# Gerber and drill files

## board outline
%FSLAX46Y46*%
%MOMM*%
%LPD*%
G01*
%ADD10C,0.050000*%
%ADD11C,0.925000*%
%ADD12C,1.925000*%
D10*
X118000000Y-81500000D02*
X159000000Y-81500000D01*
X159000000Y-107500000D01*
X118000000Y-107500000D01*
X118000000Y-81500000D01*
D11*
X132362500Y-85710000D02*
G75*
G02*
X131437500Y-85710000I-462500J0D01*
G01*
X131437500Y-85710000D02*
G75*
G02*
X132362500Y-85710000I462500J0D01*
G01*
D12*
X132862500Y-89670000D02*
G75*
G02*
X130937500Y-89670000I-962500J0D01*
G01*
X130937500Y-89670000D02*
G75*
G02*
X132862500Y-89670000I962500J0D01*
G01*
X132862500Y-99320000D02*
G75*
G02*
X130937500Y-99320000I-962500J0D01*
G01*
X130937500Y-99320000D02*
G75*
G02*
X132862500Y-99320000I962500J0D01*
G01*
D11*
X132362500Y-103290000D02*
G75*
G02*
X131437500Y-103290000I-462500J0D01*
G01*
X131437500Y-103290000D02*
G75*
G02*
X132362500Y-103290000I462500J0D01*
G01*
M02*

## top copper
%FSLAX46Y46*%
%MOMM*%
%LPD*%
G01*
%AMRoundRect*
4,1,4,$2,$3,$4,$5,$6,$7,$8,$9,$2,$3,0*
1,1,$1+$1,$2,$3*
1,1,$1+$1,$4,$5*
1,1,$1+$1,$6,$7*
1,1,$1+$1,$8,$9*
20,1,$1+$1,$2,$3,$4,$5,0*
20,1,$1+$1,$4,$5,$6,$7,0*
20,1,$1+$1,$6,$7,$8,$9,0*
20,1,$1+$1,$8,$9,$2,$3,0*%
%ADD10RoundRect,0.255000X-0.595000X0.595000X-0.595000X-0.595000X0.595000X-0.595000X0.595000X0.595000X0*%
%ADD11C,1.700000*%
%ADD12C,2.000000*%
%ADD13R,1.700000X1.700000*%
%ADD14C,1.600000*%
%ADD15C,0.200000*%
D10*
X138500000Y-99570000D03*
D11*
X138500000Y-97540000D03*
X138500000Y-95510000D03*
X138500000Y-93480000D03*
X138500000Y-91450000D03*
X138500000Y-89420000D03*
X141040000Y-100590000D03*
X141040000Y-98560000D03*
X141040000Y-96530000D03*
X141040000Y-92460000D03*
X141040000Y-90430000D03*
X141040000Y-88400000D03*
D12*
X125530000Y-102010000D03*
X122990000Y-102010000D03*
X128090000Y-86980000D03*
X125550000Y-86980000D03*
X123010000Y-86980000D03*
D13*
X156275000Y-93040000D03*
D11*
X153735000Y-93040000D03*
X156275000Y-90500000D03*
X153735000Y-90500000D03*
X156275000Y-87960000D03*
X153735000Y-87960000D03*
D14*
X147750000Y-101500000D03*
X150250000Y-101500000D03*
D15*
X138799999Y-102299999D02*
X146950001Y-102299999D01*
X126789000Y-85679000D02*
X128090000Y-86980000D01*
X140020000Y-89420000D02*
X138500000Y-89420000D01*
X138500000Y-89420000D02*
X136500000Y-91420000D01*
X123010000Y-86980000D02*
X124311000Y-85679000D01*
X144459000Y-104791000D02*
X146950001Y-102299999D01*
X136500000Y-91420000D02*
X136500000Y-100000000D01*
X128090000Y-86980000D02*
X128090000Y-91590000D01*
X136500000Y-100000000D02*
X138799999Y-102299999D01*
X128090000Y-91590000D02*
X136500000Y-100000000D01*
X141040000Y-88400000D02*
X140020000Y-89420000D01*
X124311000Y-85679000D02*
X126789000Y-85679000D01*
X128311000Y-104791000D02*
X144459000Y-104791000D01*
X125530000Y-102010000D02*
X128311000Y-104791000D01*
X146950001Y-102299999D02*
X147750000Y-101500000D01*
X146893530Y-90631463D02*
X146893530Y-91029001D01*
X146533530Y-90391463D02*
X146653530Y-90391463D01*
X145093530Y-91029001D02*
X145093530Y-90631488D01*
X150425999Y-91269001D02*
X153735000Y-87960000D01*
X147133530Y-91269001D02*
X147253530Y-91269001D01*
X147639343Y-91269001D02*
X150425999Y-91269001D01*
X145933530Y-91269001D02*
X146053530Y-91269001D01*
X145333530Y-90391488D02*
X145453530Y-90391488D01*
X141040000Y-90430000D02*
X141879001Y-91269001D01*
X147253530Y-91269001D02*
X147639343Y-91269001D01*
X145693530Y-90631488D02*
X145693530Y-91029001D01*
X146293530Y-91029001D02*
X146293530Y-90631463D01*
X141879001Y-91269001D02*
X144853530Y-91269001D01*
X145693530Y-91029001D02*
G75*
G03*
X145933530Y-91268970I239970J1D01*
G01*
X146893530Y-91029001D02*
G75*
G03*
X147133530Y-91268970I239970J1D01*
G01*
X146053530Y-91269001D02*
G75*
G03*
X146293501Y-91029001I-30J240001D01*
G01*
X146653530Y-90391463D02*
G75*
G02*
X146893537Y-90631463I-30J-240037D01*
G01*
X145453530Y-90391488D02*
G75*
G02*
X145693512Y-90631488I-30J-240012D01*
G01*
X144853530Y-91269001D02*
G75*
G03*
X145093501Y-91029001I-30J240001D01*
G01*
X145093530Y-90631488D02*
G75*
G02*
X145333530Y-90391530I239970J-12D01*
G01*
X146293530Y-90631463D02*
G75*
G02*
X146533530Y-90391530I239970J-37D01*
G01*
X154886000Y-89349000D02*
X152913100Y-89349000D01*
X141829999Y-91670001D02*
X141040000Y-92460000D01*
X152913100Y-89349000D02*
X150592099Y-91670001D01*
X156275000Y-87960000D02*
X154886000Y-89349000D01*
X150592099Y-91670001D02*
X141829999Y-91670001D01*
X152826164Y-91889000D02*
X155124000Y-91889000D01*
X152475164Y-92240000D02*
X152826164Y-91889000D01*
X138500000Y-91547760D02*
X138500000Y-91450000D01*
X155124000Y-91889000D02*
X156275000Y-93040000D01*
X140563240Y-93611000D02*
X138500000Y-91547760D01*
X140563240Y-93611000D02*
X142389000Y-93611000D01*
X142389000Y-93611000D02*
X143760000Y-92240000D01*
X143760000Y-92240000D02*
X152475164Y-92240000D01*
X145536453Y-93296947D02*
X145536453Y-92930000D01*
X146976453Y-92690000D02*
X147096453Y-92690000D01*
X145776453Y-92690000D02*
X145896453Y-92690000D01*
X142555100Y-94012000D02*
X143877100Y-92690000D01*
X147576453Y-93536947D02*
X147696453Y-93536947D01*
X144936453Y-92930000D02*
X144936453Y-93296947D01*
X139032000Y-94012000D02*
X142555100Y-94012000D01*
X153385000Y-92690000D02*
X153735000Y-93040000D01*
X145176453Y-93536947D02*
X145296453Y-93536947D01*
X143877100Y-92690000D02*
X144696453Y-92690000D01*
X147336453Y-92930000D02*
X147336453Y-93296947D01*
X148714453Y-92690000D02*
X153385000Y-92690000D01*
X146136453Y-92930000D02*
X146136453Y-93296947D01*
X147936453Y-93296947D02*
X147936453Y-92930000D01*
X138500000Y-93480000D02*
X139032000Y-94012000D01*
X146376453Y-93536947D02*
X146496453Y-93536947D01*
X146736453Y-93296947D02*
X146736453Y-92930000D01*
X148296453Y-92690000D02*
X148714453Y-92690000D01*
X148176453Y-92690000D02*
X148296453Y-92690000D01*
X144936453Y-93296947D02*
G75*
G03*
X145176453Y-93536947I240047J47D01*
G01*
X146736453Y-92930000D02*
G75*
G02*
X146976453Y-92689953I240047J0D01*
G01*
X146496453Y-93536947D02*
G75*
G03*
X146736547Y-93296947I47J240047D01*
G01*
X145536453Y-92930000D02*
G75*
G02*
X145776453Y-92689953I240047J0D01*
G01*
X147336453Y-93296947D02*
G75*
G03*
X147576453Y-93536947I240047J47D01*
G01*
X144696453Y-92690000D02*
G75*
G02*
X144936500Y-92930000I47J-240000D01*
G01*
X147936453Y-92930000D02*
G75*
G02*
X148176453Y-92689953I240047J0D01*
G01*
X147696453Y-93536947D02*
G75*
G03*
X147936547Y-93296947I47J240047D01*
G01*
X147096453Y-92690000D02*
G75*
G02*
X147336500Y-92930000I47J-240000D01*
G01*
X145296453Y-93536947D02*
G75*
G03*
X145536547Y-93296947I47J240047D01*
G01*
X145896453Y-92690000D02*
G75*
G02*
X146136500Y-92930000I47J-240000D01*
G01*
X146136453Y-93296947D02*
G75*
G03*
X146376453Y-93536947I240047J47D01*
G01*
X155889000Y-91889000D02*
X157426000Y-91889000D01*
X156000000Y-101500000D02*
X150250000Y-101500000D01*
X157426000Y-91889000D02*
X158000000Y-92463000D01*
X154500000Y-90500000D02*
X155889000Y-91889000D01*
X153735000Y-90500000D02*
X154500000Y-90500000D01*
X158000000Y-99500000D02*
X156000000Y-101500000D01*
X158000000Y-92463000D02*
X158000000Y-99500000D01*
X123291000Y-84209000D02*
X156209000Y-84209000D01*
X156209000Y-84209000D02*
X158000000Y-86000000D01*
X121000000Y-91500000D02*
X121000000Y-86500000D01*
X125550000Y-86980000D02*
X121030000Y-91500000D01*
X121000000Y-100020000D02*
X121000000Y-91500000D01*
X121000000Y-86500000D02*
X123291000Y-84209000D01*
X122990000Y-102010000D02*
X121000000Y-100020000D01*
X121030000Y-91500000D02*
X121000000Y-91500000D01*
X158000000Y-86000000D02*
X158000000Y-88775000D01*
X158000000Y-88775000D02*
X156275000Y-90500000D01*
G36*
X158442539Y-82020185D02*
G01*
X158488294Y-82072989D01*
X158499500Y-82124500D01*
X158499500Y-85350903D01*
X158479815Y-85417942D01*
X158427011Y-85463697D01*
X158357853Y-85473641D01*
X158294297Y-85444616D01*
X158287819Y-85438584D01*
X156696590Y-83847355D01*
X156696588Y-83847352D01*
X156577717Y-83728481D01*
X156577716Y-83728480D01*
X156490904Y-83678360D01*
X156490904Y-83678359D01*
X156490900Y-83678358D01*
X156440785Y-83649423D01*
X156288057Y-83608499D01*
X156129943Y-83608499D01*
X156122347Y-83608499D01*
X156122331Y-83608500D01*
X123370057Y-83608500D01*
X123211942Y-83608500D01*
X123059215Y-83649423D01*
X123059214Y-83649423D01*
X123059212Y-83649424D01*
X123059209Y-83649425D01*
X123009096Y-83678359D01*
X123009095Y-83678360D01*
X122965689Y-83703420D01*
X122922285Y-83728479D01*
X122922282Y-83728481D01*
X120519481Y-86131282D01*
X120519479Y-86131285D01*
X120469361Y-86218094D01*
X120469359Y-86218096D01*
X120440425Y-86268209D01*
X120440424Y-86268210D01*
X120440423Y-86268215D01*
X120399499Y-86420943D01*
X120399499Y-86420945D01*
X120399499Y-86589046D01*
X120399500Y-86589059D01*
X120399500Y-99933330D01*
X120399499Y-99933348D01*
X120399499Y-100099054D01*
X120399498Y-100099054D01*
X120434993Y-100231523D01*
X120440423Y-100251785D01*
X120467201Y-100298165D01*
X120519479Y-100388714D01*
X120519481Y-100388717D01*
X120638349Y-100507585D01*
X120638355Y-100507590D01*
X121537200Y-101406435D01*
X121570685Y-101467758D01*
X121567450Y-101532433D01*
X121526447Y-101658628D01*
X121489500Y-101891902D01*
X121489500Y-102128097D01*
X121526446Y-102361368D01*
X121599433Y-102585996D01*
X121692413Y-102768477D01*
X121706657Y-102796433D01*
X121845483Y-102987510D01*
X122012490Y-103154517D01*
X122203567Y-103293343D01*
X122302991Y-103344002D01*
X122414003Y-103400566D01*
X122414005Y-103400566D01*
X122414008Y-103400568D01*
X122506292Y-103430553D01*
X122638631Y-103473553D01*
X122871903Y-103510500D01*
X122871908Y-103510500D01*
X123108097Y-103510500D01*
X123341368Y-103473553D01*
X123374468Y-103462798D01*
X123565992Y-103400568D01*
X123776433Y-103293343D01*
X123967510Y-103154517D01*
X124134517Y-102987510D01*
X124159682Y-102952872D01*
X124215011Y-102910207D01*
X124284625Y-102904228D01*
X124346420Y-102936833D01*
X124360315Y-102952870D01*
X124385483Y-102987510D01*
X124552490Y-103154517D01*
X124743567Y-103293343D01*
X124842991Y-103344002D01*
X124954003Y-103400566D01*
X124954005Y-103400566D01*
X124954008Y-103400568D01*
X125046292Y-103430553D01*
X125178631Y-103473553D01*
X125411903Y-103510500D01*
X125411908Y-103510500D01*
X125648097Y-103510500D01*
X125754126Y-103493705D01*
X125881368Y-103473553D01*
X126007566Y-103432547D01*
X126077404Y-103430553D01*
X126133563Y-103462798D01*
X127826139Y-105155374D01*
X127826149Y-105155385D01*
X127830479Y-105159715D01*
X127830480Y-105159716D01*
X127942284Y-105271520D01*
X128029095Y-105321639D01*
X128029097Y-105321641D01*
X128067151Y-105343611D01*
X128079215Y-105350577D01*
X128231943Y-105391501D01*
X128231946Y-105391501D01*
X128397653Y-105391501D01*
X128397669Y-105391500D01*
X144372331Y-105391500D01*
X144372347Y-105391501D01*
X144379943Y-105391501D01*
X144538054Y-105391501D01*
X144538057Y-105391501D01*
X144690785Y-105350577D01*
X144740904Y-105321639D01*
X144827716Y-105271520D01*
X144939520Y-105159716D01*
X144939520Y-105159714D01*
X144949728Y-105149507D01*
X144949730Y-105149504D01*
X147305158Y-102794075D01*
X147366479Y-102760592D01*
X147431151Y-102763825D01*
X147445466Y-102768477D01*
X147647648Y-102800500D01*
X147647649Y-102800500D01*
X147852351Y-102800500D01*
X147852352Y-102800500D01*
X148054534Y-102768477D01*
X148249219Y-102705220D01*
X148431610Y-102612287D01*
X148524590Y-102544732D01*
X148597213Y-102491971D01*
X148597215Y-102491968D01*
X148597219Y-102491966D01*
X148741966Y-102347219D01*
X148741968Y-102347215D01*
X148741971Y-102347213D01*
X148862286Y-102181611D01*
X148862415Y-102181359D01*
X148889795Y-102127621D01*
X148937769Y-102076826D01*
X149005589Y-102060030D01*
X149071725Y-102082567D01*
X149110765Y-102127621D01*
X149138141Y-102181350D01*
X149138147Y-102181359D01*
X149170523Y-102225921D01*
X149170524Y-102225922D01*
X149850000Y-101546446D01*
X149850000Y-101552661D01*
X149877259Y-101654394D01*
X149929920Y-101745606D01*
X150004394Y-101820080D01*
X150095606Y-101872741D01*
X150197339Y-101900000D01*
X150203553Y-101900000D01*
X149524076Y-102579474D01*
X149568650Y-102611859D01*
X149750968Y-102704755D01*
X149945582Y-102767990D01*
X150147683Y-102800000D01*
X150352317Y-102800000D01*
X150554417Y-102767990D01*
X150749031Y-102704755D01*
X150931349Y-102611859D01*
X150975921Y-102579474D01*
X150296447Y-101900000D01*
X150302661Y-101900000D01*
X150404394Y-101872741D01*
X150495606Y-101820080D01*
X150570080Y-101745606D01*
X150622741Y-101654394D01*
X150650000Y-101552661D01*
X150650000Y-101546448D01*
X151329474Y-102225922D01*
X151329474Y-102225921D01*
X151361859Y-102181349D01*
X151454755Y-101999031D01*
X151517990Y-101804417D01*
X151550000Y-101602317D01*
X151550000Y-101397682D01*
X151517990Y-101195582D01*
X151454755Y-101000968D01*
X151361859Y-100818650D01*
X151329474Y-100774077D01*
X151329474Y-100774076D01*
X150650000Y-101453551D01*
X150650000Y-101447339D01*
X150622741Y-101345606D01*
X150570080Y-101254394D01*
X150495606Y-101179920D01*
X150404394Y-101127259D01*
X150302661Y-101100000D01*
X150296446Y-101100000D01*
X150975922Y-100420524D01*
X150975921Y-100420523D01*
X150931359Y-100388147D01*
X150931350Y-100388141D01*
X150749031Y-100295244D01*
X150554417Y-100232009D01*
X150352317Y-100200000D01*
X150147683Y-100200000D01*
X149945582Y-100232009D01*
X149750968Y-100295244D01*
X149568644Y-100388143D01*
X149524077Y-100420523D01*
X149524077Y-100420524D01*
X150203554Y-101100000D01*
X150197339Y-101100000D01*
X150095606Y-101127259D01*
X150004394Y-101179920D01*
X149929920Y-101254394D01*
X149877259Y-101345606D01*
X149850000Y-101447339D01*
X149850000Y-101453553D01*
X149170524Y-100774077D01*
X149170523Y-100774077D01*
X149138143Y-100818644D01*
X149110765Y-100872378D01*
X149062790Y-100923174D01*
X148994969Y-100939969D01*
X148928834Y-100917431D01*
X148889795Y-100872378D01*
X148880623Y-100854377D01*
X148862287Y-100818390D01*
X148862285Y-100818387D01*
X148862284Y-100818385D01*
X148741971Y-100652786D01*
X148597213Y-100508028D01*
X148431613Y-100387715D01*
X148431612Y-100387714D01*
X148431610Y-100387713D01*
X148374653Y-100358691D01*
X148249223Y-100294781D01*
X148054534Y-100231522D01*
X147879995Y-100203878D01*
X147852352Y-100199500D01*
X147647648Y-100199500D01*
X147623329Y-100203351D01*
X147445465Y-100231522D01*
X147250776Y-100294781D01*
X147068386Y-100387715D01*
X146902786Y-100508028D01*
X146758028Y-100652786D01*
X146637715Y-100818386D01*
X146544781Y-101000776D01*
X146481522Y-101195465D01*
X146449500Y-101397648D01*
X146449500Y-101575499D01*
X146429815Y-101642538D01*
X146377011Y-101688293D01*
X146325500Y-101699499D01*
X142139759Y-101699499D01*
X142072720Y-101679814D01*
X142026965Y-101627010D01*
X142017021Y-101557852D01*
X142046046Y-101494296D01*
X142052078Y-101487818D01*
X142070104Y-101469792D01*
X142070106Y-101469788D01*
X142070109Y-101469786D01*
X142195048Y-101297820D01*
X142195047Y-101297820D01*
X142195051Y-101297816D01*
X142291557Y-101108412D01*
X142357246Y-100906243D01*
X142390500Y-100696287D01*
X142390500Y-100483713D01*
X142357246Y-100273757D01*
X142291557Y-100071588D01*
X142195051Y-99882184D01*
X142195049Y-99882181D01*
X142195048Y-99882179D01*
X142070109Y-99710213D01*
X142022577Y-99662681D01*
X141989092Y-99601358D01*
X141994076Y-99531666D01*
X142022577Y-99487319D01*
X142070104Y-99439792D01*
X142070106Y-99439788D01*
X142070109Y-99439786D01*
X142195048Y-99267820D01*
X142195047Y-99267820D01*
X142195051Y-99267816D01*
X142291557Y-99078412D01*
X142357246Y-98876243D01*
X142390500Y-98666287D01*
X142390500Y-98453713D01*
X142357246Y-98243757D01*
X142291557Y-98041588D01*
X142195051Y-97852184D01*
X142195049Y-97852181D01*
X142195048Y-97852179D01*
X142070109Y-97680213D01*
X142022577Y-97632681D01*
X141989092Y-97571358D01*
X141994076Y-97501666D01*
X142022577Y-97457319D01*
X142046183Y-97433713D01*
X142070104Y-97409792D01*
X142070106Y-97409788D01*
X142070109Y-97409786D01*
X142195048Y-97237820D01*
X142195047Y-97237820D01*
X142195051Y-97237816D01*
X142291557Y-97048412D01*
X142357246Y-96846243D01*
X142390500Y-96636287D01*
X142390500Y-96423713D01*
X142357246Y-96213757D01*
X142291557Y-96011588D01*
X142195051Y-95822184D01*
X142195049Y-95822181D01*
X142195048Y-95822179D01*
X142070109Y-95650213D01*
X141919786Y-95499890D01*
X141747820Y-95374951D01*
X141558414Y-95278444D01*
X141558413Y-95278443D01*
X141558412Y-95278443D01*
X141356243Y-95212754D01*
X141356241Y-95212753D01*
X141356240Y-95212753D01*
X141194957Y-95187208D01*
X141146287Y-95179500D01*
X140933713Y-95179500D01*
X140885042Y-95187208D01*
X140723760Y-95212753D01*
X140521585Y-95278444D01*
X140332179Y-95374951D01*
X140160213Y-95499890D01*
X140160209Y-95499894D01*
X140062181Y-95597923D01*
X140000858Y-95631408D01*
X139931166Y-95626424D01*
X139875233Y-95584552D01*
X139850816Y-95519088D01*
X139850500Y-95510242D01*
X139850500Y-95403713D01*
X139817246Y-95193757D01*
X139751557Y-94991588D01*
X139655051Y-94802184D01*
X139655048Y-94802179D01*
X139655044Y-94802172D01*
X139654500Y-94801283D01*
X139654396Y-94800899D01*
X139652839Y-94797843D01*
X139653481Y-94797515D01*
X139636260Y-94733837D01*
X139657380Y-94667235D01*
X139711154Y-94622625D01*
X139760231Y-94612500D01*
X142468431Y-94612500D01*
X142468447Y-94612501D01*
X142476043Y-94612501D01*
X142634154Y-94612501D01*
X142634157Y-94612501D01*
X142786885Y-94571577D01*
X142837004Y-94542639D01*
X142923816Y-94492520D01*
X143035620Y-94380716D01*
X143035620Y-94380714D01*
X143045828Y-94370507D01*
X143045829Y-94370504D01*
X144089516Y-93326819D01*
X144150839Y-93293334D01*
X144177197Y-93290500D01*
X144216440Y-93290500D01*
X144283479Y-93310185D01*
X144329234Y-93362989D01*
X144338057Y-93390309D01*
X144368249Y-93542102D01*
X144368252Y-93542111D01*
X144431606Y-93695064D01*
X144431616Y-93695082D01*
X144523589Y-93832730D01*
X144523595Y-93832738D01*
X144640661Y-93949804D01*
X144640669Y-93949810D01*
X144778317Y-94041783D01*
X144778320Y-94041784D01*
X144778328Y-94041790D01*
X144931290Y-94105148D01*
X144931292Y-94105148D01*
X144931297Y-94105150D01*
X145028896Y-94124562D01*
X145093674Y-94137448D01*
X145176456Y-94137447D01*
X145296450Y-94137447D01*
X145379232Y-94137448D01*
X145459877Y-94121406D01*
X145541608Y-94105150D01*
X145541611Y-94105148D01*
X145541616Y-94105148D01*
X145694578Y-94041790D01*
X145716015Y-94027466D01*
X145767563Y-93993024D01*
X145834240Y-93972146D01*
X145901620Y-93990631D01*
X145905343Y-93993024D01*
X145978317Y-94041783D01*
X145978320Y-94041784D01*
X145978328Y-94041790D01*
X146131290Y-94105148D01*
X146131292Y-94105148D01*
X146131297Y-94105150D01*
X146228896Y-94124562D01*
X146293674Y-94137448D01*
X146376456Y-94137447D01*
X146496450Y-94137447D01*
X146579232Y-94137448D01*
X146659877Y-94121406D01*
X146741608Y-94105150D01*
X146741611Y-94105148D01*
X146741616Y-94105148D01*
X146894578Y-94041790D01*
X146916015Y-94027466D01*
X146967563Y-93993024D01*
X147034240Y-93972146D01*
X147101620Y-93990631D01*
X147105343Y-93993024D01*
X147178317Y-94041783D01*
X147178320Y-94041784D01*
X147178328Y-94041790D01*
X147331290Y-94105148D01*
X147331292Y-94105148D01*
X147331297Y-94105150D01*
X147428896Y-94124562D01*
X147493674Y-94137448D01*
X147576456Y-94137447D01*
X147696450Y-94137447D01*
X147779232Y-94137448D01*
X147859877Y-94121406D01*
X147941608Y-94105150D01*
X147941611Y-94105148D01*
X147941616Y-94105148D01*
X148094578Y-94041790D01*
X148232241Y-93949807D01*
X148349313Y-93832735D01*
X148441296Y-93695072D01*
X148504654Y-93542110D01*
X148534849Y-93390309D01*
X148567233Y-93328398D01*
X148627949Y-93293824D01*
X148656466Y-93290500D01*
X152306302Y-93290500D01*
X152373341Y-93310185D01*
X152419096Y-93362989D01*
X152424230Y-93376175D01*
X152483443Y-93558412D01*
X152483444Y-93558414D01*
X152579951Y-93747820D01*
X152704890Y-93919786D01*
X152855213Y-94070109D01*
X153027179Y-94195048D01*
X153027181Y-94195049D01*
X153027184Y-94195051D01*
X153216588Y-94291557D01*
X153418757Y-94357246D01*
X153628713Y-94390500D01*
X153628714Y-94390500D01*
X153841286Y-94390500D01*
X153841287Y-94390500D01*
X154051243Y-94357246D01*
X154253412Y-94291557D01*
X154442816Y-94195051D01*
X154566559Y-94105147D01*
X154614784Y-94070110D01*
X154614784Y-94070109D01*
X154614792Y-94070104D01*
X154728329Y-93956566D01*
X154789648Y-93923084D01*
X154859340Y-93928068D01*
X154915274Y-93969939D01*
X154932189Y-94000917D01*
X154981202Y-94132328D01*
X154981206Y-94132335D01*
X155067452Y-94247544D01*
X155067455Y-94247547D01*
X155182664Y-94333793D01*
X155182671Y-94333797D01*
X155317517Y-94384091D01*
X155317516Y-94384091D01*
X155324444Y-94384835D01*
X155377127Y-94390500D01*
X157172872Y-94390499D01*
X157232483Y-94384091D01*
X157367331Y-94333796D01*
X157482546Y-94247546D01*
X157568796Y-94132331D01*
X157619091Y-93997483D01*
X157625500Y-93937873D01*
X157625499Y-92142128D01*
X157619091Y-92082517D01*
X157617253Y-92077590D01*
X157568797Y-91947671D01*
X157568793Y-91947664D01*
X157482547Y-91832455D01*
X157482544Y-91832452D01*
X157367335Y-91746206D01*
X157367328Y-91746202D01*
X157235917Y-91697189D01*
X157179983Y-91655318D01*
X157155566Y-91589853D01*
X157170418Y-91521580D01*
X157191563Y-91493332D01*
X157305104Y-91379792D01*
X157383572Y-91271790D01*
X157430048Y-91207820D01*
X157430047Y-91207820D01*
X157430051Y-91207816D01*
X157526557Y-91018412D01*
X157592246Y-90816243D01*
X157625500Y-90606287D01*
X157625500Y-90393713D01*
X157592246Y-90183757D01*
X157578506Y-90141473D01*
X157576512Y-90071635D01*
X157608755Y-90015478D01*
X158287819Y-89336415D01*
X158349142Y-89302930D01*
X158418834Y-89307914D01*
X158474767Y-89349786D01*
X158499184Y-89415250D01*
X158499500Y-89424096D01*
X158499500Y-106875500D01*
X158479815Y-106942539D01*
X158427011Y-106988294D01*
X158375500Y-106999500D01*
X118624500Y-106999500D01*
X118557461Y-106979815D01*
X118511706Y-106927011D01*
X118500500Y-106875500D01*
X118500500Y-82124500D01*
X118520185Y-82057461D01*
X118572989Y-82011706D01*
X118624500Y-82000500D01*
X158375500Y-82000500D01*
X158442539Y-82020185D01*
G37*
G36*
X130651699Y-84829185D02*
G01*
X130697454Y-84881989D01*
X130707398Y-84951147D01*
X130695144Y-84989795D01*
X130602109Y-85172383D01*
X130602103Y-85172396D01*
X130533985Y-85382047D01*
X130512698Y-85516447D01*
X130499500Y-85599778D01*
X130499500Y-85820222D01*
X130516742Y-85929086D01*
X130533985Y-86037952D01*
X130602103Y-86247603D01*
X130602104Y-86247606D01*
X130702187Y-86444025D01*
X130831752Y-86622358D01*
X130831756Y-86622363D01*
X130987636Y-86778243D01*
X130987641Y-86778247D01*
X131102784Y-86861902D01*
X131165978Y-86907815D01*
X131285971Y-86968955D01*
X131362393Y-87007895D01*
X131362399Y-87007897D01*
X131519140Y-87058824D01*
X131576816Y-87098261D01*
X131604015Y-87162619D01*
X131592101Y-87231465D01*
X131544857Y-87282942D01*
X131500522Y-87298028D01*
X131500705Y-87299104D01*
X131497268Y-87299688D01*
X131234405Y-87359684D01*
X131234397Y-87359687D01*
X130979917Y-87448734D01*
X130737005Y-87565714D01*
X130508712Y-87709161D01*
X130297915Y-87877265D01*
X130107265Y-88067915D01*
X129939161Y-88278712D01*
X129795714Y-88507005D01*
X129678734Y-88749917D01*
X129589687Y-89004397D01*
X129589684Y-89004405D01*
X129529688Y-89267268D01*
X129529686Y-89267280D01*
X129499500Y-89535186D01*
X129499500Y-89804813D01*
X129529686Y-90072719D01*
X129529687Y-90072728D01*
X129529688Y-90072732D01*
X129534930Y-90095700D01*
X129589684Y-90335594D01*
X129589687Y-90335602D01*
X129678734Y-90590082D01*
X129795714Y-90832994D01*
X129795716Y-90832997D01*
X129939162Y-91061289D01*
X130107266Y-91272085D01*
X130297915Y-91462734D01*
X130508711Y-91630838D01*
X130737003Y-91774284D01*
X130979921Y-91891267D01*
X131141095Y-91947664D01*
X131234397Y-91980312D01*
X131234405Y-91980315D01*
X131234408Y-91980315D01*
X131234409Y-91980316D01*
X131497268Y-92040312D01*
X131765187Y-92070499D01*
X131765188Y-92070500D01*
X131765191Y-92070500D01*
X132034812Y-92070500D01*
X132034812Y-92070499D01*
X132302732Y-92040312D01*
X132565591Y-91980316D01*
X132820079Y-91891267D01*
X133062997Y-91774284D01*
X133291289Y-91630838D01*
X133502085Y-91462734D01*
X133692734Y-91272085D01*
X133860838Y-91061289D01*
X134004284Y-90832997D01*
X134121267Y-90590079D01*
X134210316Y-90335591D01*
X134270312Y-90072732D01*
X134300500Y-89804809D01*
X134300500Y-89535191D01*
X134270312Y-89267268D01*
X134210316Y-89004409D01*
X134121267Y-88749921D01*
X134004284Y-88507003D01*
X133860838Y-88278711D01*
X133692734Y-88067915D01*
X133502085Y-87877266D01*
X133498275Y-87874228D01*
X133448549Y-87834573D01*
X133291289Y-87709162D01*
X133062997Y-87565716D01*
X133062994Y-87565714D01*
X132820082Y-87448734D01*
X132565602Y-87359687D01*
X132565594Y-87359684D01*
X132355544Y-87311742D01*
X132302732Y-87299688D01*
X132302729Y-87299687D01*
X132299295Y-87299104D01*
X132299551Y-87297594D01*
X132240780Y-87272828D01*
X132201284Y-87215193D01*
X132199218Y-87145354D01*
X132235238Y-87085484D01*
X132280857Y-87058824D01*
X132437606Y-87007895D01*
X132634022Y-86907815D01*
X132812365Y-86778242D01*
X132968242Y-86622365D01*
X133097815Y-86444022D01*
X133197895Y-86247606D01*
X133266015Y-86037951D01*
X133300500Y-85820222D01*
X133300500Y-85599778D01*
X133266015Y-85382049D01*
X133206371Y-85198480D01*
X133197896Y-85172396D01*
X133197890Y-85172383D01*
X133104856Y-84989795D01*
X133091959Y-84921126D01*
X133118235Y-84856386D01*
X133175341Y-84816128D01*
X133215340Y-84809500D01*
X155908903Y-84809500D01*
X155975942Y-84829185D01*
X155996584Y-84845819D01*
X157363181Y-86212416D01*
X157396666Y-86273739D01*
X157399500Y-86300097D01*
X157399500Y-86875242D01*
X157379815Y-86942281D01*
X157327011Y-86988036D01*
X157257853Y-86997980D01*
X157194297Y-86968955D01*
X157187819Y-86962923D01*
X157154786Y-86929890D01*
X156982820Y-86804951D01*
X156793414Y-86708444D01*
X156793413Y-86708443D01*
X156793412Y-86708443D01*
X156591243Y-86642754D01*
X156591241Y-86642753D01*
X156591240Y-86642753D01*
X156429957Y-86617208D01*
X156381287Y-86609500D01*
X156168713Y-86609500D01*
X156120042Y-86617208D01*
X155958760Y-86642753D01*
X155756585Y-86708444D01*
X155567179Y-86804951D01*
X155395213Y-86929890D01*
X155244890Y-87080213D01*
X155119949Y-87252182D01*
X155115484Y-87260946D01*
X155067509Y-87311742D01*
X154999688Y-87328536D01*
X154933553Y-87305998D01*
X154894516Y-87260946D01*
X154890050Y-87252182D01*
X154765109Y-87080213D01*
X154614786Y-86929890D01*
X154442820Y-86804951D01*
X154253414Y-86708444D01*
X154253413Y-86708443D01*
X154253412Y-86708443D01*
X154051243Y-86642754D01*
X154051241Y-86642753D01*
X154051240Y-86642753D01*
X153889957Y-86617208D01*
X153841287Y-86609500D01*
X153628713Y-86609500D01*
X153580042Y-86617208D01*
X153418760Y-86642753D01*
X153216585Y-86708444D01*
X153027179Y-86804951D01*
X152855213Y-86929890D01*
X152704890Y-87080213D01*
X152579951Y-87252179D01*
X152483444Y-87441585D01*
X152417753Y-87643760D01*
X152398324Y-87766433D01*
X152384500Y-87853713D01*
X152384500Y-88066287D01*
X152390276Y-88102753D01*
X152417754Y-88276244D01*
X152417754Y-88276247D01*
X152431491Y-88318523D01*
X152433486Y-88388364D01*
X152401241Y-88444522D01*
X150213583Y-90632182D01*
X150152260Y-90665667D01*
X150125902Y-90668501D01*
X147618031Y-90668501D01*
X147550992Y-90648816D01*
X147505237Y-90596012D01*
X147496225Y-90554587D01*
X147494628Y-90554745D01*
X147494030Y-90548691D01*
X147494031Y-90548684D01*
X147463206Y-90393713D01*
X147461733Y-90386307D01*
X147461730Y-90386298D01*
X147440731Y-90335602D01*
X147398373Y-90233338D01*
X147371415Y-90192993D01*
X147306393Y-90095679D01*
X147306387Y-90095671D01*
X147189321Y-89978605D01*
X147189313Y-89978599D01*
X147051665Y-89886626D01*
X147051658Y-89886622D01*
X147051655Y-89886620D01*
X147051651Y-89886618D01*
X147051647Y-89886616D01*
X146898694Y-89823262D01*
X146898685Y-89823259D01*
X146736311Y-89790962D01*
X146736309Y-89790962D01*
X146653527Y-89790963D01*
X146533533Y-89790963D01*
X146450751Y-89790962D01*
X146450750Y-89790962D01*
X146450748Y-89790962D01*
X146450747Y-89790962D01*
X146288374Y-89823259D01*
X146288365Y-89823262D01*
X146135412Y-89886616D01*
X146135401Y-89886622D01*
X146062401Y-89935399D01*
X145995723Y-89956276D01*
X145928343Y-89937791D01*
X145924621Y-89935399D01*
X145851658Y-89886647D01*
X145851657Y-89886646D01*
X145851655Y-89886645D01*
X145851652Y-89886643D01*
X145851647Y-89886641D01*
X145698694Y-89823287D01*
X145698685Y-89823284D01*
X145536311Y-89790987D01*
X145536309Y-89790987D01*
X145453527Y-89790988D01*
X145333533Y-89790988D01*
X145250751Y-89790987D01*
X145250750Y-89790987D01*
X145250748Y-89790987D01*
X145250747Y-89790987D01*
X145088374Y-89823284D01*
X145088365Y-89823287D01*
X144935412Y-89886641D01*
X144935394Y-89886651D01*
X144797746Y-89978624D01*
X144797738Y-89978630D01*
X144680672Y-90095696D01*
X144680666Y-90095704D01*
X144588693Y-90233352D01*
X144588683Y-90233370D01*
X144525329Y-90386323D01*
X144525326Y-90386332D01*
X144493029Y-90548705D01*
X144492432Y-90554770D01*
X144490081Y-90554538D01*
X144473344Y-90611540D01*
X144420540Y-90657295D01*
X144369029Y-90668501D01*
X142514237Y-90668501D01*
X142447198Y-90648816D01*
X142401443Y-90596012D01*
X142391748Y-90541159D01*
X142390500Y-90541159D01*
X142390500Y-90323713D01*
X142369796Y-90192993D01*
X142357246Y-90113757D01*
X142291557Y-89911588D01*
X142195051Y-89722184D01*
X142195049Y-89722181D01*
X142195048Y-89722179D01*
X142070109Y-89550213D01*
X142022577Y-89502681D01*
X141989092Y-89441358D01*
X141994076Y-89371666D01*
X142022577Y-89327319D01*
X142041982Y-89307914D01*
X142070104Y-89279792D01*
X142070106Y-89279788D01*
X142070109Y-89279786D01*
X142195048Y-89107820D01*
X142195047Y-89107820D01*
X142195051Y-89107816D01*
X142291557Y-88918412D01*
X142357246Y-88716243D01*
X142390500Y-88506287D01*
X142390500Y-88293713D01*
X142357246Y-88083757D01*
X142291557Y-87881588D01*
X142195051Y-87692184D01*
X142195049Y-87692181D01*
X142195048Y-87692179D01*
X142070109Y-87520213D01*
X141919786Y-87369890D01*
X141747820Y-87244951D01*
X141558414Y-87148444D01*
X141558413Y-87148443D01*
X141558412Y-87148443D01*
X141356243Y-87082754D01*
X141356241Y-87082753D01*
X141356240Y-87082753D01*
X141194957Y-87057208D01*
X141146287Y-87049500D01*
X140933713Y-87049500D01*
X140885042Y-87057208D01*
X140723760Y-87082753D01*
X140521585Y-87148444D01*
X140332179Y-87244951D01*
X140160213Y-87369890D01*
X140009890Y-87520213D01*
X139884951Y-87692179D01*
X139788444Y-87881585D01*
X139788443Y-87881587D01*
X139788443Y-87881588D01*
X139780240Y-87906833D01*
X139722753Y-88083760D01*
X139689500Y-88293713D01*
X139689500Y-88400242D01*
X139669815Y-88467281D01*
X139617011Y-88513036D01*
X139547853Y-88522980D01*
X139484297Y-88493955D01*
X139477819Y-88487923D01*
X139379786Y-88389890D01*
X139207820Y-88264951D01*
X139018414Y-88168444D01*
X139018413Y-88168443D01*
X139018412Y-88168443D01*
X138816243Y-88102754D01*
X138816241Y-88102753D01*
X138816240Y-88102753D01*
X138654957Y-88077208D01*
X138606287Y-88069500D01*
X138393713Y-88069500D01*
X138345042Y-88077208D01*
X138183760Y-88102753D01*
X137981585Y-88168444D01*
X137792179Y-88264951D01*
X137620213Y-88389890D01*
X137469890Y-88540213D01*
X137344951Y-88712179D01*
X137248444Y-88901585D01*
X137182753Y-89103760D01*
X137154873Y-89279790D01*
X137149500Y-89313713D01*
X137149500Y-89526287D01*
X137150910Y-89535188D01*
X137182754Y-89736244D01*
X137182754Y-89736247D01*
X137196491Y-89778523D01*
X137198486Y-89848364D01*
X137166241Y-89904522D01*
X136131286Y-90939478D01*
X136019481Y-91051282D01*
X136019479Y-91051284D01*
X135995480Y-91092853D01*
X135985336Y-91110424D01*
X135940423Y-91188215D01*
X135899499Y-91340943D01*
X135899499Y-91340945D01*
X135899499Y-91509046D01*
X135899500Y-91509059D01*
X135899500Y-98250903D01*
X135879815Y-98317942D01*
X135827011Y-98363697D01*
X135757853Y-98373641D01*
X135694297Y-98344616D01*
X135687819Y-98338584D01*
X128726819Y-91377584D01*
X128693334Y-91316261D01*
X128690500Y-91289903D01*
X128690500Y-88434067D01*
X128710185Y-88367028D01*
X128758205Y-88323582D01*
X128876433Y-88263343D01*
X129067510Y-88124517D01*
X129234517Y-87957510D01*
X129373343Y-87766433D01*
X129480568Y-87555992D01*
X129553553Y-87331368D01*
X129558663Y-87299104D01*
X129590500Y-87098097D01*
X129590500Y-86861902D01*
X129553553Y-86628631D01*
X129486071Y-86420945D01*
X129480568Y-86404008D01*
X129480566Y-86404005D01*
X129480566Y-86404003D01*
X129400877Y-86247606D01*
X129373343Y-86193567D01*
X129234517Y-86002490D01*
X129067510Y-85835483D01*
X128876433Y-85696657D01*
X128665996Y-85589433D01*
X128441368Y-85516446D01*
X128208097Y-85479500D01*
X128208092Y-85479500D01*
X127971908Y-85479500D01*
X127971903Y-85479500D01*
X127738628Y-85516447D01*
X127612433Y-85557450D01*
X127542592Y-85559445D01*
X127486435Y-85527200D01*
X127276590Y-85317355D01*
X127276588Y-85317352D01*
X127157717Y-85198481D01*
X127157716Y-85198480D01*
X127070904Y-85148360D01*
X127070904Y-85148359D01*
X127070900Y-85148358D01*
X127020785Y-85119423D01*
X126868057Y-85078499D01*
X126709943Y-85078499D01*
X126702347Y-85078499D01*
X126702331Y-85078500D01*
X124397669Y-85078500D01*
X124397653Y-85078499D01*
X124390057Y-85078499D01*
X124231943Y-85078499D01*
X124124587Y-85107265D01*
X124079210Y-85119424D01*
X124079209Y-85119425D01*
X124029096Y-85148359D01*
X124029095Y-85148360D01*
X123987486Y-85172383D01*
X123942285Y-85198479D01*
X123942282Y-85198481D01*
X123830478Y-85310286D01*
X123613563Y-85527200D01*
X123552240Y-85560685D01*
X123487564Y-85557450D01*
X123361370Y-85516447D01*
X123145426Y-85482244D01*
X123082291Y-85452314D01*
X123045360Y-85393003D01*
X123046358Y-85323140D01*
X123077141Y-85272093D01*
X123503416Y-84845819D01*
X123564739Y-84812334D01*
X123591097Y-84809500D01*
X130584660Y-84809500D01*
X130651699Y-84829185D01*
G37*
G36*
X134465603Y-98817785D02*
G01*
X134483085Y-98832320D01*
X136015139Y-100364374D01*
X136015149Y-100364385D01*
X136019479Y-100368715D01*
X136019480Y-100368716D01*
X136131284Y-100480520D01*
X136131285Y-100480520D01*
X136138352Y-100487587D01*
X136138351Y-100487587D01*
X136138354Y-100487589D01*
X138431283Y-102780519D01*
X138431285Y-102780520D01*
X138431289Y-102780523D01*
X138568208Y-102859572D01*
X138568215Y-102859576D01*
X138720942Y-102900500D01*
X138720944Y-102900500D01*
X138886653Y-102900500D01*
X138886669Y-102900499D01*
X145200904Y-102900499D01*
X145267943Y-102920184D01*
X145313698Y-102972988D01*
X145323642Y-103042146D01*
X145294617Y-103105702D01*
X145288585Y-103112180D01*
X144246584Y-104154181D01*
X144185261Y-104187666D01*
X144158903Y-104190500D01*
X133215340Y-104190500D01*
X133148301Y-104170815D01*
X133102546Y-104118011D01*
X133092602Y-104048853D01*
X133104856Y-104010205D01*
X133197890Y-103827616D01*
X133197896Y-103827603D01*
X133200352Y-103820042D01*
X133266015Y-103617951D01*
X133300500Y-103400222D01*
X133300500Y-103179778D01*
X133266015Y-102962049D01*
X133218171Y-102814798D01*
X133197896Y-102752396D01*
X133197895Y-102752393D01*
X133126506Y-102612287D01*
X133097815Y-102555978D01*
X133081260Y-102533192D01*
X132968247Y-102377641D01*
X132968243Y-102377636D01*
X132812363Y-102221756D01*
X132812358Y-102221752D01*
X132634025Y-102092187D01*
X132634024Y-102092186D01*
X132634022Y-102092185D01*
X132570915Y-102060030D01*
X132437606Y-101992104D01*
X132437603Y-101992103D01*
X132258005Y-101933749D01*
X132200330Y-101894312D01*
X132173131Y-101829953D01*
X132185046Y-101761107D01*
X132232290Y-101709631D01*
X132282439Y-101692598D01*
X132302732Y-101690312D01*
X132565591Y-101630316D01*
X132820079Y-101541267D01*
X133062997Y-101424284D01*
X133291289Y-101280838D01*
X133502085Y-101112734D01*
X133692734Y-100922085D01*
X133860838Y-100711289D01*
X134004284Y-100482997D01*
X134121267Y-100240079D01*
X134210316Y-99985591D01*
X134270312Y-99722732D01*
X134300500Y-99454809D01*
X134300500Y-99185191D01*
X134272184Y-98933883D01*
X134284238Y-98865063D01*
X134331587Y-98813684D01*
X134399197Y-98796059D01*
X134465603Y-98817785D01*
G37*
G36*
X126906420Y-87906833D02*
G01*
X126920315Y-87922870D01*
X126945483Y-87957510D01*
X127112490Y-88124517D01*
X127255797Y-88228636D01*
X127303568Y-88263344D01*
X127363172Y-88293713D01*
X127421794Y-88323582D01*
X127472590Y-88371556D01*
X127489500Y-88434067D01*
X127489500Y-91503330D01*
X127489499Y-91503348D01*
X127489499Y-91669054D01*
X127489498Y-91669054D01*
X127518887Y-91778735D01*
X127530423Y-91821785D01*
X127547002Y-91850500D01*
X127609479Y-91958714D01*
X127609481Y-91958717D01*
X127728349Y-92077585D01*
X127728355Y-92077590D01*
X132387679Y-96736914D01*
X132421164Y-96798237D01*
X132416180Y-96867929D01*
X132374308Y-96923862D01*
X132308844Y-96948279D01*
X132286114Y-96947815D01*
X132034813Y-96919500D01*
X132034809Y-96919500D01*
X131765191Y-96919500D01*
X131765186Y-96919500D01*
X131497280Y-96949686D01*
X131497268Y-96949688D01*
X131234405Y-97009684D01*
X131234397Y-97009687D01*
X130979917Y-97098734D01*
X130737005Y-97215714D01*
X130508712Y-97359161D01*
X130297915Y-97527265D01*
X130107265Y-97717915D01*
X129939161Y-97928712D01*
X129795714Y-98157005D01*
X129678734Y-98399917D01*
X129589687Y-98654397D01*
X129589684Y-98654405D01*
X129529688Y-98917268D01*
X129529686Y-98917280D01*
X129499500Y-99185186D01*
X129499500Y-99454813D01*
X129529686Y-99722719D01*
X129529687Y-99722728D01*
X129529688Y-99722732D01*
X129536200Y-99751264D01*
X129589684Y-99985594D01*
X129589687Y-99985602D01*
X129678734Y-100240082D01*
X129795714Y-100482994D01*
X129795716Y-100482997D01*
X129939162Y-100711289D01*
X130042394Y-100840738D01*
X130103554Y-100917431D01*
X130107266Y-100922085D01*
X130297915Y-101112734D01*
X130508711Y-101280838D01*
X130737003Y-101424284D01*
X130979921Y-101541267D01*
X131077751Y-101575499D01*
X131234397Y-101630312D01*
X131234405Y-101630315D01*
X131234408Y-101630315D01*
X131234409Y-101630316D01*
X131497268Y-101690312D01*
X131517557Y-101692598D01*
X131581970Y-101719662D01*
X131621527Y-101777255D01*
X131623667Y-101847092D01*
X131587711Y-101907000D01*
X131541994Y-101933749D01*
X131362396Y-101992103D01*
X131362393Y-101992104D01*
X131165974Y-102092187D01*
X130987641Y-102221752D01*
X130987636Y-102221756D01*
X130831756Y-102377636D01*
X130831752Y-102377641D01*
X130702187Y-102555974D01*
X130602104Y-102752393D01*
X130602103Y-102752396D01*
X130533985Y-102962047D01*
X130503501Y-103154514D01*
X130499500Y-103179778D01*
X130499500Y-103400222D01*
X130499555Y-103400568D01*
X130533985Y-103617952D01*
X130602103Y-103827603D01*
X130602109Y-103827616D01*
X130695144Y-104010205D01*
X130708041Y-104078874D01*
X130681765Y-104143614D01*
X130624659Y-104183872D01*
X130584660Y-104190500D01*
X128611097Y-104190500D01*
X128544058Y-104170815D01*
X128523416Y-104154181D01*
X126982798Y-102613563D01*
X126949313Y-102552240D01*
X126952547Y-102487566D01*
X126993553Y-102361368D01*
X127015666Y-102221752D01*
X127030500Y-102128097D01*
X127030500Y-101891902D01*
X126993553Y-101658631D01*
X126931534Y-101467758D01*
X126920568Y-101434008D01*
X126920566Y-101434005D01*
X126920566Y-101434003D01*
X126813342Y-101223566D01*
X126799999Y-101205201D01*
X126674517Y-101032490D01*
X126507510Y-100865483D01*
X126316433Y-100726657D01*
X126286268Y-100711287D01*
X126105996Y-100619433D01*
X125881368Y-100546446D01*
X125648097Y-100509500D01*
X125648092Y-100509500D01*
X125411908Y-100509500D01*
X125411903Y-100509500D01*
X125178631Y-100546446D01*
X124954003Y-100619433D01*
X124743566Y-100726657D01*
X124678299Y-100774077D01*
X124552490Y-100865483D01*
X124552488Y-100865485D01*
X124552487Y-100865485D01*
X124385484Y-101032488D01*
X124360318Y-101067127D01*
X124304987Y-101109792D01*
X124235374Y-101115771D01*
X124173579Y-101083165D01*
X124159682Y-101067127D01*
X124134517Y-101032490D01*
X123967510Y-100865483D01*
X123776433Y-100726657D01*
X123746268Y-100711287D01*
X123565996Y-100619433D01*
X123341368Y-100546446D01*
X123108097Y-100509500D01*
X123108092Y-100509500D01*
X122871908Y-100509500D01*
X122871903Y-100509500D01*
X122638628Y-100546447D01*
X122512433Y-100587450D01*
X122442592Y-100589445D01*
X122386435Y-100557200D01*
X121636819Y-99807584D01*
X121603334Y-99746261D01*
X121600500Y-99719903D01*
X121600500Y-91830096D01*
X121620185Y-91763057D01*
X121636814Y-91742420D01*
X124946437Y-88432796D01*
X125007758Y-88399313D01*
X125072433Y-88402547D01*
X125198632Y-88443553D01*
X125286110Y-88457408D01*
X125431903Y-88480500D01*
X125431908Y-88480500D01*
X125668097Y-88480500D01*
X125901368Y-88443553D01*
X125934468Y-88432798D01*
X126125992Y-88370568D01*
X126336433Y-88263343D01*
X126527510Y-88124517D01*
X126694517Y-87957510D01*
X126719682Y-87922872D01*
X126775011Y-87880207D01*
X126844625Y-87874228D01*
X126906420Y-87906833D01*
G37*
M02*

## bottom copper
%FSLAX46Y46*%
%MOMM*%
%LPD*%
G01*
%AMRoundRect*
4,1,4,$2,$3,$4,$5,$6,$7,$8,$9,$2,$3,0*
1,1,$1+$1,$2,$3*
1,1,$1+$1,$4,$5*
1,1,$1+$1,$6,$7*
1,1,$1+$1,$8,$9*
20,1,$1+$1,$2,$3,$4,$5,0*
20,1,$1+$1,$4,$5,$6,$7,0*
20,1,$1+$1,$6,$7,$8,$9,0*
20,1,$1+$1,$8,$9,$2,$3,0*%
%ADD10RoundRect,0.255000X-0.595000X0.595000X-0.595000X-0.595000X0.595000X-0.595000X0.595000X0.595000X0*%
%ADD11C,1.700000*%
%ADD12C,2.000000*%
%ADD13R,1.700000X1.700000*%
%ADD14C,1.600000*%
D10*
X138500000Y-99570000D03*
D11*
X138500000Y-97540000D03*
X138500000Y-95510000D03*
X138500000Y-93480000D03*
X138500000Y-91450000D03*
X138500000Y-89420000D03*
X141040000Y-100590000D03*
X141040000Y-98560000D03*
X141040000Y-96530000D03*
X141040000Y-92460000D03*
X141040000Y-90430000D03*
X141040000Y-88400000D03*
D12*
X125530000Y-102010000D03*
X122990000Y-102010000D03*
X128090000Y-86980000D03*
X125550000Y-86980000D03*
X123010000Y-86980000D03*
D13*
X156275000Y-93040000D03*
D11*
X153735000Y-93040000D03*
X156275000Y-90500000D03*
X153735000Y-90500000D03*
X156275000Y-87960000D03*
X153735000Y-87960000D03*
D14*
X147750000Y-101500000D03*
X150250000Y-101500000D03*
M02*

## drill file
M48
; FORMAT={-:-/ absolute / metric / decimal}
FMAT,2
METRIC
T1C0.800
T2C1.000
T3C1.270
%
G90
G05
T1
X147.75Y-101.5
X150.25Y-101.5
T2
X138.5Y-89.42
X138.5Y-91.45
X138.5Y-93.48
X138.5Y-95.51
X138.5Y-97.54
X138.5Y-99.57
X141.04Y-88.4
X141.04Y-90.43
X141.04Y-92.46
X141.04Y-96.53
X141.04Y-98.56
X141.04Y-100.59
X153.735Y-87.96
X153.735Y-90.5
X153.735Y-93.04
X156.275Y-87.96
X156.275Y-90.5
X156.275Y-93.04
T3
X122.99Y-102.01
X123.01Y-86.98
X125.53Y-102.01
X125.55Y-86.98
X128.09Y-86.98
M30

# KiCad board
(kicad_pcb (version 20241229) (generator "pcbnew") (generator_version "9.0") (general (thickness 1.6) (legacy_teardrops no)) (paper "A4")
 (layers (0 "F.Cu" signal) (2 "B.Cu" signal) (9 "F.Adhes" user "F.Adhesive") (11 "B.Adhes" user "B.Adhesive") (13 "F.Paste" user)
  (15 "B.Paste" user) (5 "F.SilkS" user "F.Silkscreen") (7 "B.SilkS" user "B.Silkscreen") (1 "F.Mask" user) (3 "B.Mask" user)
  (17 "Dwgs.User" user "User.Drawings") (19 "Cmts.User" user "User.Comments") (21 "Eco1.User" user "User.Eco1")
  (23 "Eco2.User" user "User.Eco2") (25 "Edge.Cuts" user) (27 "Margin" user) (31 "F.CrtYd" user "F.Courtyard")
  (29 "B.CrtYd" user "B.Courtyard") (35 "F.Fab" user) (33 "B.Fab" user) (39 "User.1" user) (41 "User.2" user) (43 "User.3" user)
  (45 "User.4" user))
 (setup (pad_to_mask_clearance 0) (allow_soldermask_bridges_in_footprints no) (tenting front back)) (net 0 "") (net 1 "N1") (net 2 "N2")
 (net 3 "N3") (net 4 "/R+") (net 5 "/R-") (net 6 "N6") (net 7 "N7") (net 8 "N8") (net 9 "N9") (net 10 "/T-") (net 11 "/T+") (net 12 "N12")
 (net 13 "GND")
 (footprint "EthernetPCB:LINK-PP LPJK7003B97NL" (layer "F.Cu") (at 138.5 99.57 -90)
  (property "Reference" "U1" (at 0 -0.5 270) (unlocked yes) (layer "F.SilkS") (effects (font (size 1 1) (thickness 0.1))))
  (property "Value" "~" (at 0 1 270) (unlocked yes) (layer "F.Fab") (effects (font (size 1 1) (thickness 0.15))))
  (fp_circle (center -13.86 6.6) (end -12.96 6.6) (stroke (width 0.05) (type solid)) (fill yes) (layer "Edge.Cuts"))
  (fp_circle (center -9.9 6.6) (end -8 6.6) (stroke (width 0.05) (type solid)) (fill yes) (layer "Edge.Cuts"))
  (fp_circle (center -0.25 6.6) (end 1.65 6.6) (stroke (width 0.05) (type solid)) (fill yes) (layer "Edge.Cuts"))
  (fp_circle (center 3.72 6.6) (end 4.62 6.6) (stroke (width 0.05) (type solid)) (fill yes) (layer "Edge.Cuts"))
  (pad "1" thru_hole roundrect (at 0 0 270) (size 1.7 1.7) (drill 1) (layers "*.Cu" "*.Mask") (remove_unused_layers no)
   (roundrect_rratio 0.15) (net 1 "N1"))
  (pad "2" thru_hole circle (at -2.03 0 270) (size 1.7 1.7) (drill 1) (layers "*.Cu" "*.Mask") (remove_unused_layers no) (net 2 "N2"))
  (pad "3" thru_hole circle (at -4.06 0 270) (size 1.7 1.7) (drill 1) (layers "*.Cu" "*.Mask") (remove_unused_layers no) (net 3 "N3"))
  (pad "4" thru_hole circle (at -6.09 0 270) (size 1.7 1.7) (drill 1) (layers "*.Cu" "*.Mask") (remove_unused_layers no) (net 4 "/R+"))
  (pad "5" thru_hole circle (at -8.12 0 270) (size 1.7 1.7) (drill 1) (layers "*.Cu" "*.Mask") (remove_unused_layers no) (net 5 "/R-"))
  (pad "6" thru_hole circle (at -10.15 0 270) (size 1.7 1.7) (drill 1) (layers "*.Cu" "*.Mask") (remove_unused_layers no) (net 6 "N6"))
  (pad "7" thru_hole circle (at 1.02 -2.54 270) (size 1.7 1.7) (drill 1) (layers "*.Cu" "*.Mask") (remove_unused_layers no) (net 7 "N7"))
  (pad "8" thru_hole circle (at -1.01 -2.54 270) (size 1.7 1.7) (drill 1) (layers "*.Cu" "*.Mask") (remove_unused_layers no) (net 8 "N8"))
  (pad "9" thru_hole circle (at -3.04 -2.54 270) (size 1.7 1.7) (drill 1) (layers "*.Cu" "*.Mask") (remove_unused_layers no) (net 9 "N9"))
  (pad "10" thru_hole circle (at -7.11 -2.54 270) (size 1.7 1.7) (drill 1) (layers "*.Cu" "*.Mask") (remove_unused_layers no) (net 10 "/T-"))
  (pad "11" thru_hole circle (at -9.14 -2.54 270) (size 1.7 1.7) (drill 1) (layers "*.Cu" "*.Mask") (remove_unused_layers no) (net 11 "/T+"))
  (pad "12" thru_hole circle (at -11.17 -2.54 270) (size 1.7 1.7) (drill 1) (layers "*.Cu" "*.Mask") (remove_unused_layers no) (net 6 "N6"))
  (pad "13" thru_hole circle (at 2.44 12.97 270) (size 2 2) (drill 1.27) (layers "*.Cu" "*.Mask") (remove_unused_layers no) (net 6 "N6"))
  (pad "14" thru_hole circle (at 2.44 15.51 270) (size 2 2) (drill 1.27) (layers "*.Cu" "*.Mask") (remove_unused_layers no) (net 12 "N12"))
  (pad "15" thru_hole circle (at -12.59 10.41 270) (size 2 2) (drill 1.27) (layers "*.Cu" "*.Mask") (remove_unused_layers no) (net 6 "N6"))
  (pad "16" thru_hole circle (at -12.59 12.95 270) (size 2 2) (drill 1.27) (layers "*.Cu" "*.Mask") (remove_unused_layers no) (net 12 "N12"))
  (pad "17" thru_hole circle (at -12.59 15.49 270) (size 2 2) (drill 1.27) (layers "*.Cu" "*.Mask") (remove_unused_layers no) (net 6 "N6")))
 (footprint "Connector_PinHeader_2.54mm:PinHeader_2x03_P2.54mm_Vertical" (layer "F.Cu") (at 156.275 93.04 180)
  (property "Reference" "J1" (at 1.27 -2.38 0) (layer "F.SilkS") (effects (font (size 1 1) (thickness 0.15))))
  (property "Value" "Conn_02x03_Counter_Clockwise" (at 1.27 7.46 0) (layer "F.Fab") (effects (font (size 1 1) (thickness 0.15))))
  (pad "1" thru_hole rect (at 0 0 180) (size 1.7 1.7) (drill 1) (layers "*.Cu" "*.Mask") (remove_unused_layers no) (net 5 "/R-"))
  (pad "2" thru_hole circle (at 2.54 0 180) (size 1.7 1.7) (drill 1) (layers "*.Cu" "*.Mask") (remove_unused_layers no) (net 4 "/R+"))
  (pad "3" thru_hole circle (at 0 2.54 180) (size 1.7 1.7) (drill 1) (layers "*.Cu" "*.Mask") (remove_unused_layers no) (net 12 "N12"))
  (pad "4" thru_hole circle (at 2.54 2.54 180) (size 1.7 1.7) (drill 1) (layers "*.Cu" "*.Mask") (remove_unused_layers no) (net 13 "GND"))
  (pad "5" thru_hole circle (at 0 5.08 180) (size 1.7 1.7) (drill 1) (layers "*.Cu" "*.Mask") (remove_unused_layers no) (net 10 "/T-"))
  (pad "6" thru_hole circle (at 2.54 5.08 180) (size 1.7 1.7) (drill 1) (layers "*.Cu" "*.Mask") (remove_unused_layers no) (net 11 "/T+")))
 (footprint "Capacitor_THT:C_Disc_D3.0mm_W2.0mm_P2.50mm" (layer "F.Cu") (at 147.75 101.5)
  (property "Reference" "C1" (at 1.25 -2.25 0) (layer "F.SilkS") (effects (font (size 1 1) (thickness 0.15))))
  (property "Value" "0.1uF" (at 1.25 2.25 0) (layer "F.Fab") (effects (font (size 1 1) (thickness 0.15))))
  (pad "1" thru_hole circle (at 0 0) (size 1.6 1.6) (drill 0.8) (layers "*.Cu" "*.Mask") (remove_unused_layers no) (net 6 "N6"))
  (pad "2" thru_hole circle (at 2.5 0) (size 1.6 1.6) (drill 0.8) (layers "*.Cu" "*.Mask") (remove_unused_layers no) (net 13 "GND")))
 (gr_rect (start 118 81.5) (end 159 107.5) (stroke (width 0.05) (type solid)) (fill no) (layer "Edge.Cuts"))
 (segment (start 138.799999 102.299999) (end 146.950001 102.299999) (width 0.2) (layer "F.Cu") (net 6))
 (segment (start 126.789 85.679) (end 128.09 86.98) (width 0.2) (layer "F.Cu") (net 6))
 (segment (start 140.02 89.42) (end 138.5 89.42) (width 0.2) (layer "F.Cu") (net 6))
 (segment (start 138.5 89.42) (end 136.5 91.42) (width 0.2) (layer "F.Cu") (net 6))
 (segment (start 123.01 86.98) (end 124.311 85.679) (width 0.2) (layer "F.Cu") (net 6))
 (segment (start 144.459 104.791) (end 146.950001 102.299999) (width 0.2) (layer "F.Cu") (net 6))
 (segment (start 136.5 91.42) (end 136.5 100) (width 0.2) (layer "F.Cu") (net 6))
 (segment (start 128.09 86.98) (end 128.09 91.59) (width 0.2) (layer "F.Cu") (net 6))
 (segment (start 136.5 100) (end 138.799999 102.299999) (width 0.2) (layer "F.Cu") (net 6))
 (segment (start 128.09 91.59) (end 136.5 100) (width 0.2) (layer "F.Cu") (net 6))
 (segment (start 141.04 88.4) (end 140.02 89.42) (width 0.2) (layer "F.Cu") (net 6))
 (segment (start 124.311 85.679) (end 126.789 85.679) (width 0.2) (layer "F.Cu") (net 6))
 (segment (start 128.311 104.791) (end 144.459 104.791) (width 0.2) (layer "F.Cu") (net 6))
 (segment (start 125.53 102.01) (end 128.311 104.791) (width 0.2) (layer "F.Cu") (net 6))
 (segment (start 146.950001 102.299999) (end 147.75 101.5) (width 0.2) (layer "F.Cu") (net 6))
 (segment (start 146.89353 90.631463) (end 146.89353 91.029001) (width 0.2) (layer "F.Cu") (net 11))
 (segment (start 146.53353 90.391463) (end 146.65353 90.391463) (width 0.2) (layer "F.Cu") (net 11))
 (segment (start 145.09353 91.029001) (end 145.09353 90.631488) (width 0.2) (layer "F.Cu") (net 11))
 (segment (start 150.425999 91.269001) (end 153.735 87.96) (width 0.2) (layer "F.Cu") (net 11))
 (segment (start 147.13353 91.269001) (end 147.25353 91.269001) (width 0.2) (layer "F.Cu") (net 11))
 (segment (start 147.639343 91.269001) (end 150.425999 91.269001) (width 0.2) (layer "F.Cu") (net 11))
 (segment (start 145.93353 91.269001) (end 146.05353 91.269001) (width 0.2) (layer "F.Cu") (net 11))
 (segment (start 145.33353 90.391488) (end 145.45353 90.391488) (width 0.2) (layer "F.Cu") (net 11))
 (segment (start 141.04 90.43) (end 141.879001 91.269001) (width 0.2) (layer "F.Cu") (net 11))
 (segment (start 147.25353 91.269001) (end 147.639343 91.269001) (width 0.2) (layer "F.Cu") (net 11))
 (segment (start 145.69353 90.631488) (end 145.69353 91.029001) (width 0.2) (layer "F.Cu") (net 11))
 (segment (start 146.29353 91.029001) (end 146.29353 90.631463) (width 0.2) (layer "F.Cu") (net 11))
 (segment (start 141.879001 91.269001) (end 144.85353 91.269001) (width 0.2) (layer "F.Cu") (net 11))
 (arc (start 145.69353 91.029001) (mid 145.763824 91.198707) (end 145.93353 91.269001) (width 0.2) (layer "F.Cu") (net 11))
 (arc (start 146.89353 91.029001) (mid 146.963824 91.198707) (end 147.13353 91.269001) (width 0.2) (layer "F.Cu") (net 11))
 (arc (start 146.05353 91.269001) (mid 146.223236 91.198707) (end 146.29353 91.029001) (width 0.2) (layer "F.Cu") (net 11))
 (arc (start 146.65353 90.391463) (mid 146.823236 90.461757) (end 146.89353 90.631463) (width 0.2) (layer "F.Cu") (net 11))
 (arc (start 145.45353 90.391488) (mid 145.623236 90.461782) (end 145.69353 90.631488) (width 0.2) (layer "F.Cu") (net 11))
 (arc (start 144.85353 91.269001) (mid 145.023236 91.198707) (end 145.09353 91.029001) (width 0.2) (layer "F.Cu") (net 11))
 (arc (start 145.09353 90.631488) (mid 145.163824 90.461782) (end 145.33353 90.391488) (width 0.2) (layer "F.Cu") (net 11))
 (arc (start 146.29353 90.631463) (mid 146.363824 90.461757) (end 146.53353 90.391463) (width 0.2) (layer "F.Cu") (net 11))
 (segment (start 154.886 89.349) (end 152.9131 89.349) (width 0.2) (layer "F.Cu") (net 10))
 (segment (start 141.829999 91.670001) (end 141.04 92.46) (width 0.2) (layer "F.Cu") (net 10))
 (segment (start 152.9131 89.349) (end 150.592099 91.670001) (width 0.2) (layer "F.Cu") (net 10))
 (segment (start 156.275 87.96) (end 154.886 89.349) (width 0.2) (layer "F.Cu") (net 10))
 (segment (start 150.592099 91.670001) (end 141.829999 91.670001) (width 0.2) (layer "F.Cu") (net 10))
 (segment (start 152.826164 91.889) (end 155.124 91.889) (width 0.2) (layer "F.Cu") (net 5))
 (segment (start 152.475164 92.24) (end 152.826164 91.889) (width 0.2) (layer "F.Cu") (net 5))
 (segment (start 138.5 91.54776) (end 138.5 91.45) (width 0.2) (layer "F.Cu") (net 5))
 (segment (start 155.124 91.889) (end 156.275 93.04) (width 0.2) (layer "F.Cu") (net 5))
 (segment (start 140.56324 93.611) (end 138.5 91.54776) (width 0.2) (layer "F.Cu") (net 5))
 (segment (start 140.56324 93.611) (end 142.389 93.611) (width 0.2) (layer "F.Cu") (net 5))
 (segment (start 142.389 93.611) (end 143.76 92.24) (width 0.2) (layer "F.Cu") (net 5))
 (segment (start 143.76 92.24) (end 152.475164 92.24) (width 0.2) (layer "F.Cu") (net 5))
 (segment (start 145.536453 93.296947) (end 145.536453 92.93) (width 0.2) (layer "F.Cu") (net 4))
 (segment (start 146.976453 92.69) (end 147.096453 92.69) (width 0.2) (layer "F.Cu") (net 4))
 (segment (start 145.776453 92.69) (end 145.896453 92.69) (width 0.2) (layer "F.Cu") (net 4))
 (segment (start 142.5551 94.012) (end 143.8771 92.69) (width 0.2) (layer "F.Cu") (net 4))
 (segment (start 147.576453 93.536947) (end 147.696453 93.536947) (width 0.2) (layer "F.Cu") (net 4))
 (segment (start 144.936453 92.93) (end 144.936453 93.296947) (width 0.2) (layer "F.Cu") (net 4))
 (segment (start 139.032 94.012) (end 142.5551 94.012) (width 0.2) (layer "F.Cu") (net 4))
 (segment (start 153.385 92.69) (end 153.735 93.04) (width 0.2) (layer "F.Cu") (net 4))
 (segment (start 145.176453 93.536947) (end 145.296453 93.536947) (width 0.2) (layer "F.Cu") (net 4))
 (segment (start 143.8771 92.69) (end 144.696453 92.69) (width 0.2) (layer "F.Cu") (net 4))
 (segment (start 147.336453 92.93) (end 147.336453 93.296947) (width 0.2) (layer "F.Cu") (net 4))
 (segment (start 148.714453 92.69) (end 153.385 92.69) (width 0.2) (layer "F.Cu") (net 4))
 (segment (start 146.136453 92.93) (end 146.136453 93.296947) (width 0.2) (layer "F.Cu") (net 4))
 (segment (start 147.936453 93.296947) (end 147.936453 92.93) (width 0.2) (layer "F.Cu") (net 4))
 (segment (start 138.5 93.48) (end 139.032 94.012) (width 0.2) (layer "F.Cu") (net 4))
 (segment (start 146.376453 93.536947) (end 146.496453 93.536947) (width 0.2) (layer "F.Cu") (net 4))
 (segment (start 146.736453 93.296947) (end 146.736453 92.93) (width 0.2) (layer "F.Cu") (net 4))
 (segment (start 148.296453 92.69) (end 148.714453 92.69) (width 0.2) (layer "F.Cu") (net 4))
 (segment (start 148.176453 92.69) (end 148.296453 92.69) (width 0.2) (layer "F.Cu") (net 4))
 (arc (start 144.936453 93.296947) (mid 145.006747 93.466653) (end 145.176453 93.536947) (width 0.2) (layer "F.Cu") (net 4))
 (arc (start 146.736453 92.93) (mid 146.806747 92.760294) (end 146.976453 92.69) (width 0.2) (layer "F.Cu") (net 4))
 (arc (start 146.496453 93.536947) (mid 146.666159 93.466653) (end 146.736453 93.296947) (width 0.2) (layer "F.Cu") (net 4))
 (arc (start 145.536453 92.93) (mid 145.606747 92.760294) (end 145.776453 92.69) (width 0.2) (layer "F.Cu") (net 4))
 (arc (start 147.336453 93.296947) (mid 147.406747 93.466653) (end 147.576453 93.536947) (width 0.2) (layer "F.Cu") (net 4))
 (arc (start 144.696453 92.69) (mid 144.866159 92.760294) (end 144.936453 92.93) (width 0.2) (layer "F.Cu") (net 4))
 (arc (start 147.936453 92.93) (mid 148.006747 92.760294) (end 148.176453 92.69) (width 0.2) (layer "F.Cu") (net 4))
 (arc (start 147.696453 93.536947) (mid 147.866159 93.466653) (end 147.936453 93.296947) (width 0.2) (layer "F.Cu") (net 4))
 (arc (start 147.096453 92.69) (mid 147.266159 92.760294) (end 147.336453 92.93) (width 0.2) (layer "F.Cu") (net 4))
 (arc (start 145.296453 93.536947) (mid 145.466159 93.466653) (end 145.536453 93.296947) (width 0.2) (layer "F.Cu") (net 4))
 (arc (start 145.896453 92.69) (mid 146.066159 92.760294) (end 146.136453 92.93) (width 0.2) (layer "F.Cu") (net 4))
 (arc (start 146.136453 93.296947) (mid 146.206747 93.466653) (end 146.376453 93.536947) (width 0.2) (layer "F.Cu") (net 4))
 (segment (start 155.889 91.889) (end 157.426 91.889) (width 0.2) (layer "F.Cu") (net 13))
 (segment (start 156 101.5) (end 150.25 101.5) (width 0.2) (layer "F.Cu") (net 13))
 (segment (start 157.426 91.889) (end 158 92.463) (width 0.2) (layer "F.Cu") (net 13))
 (segment (start 154.5 90.5) (end 155.889 91.889) (width 0.2) (layer "F.Cu") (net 13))
 (segment (start 153.735 90.5) (end 154.5 90.5) (width 0.2) (layer "F.Cu") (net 13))
 (segment (start 158 99.5) (end 156 101.5) (width 0.2) (layer "F.Cu") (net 13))
 (segment (start 158 92.463) (end 158 99.5) (width 0.2) (layer "F.Cu") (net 13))
 (segment (start 123.291 84.209) (end 156.209 84.209) (width 0.2) (layer "F.Cu") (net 12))
 (segment (start 156.209 84.209) (end 158 86) (width 0.2) (layer "F.Cu") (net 12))
 (segment (start 121 91.5) (end 121 86.5) (width 0.2) (layer "F.Cu") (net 12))
 (segment (start 125.55 86.98) (end 121.03 91.5) (width 0.2) (layer "F.Cu") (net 12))
 (segment (start 121 100.02) (end 121 91.5) (width 0.2) (layer "F.Cu") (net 12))
 (segment (start 121 86.5) (end 123.291 84.209) (width 0.2) (layer "F.Cu") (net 12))
 (segment (start 122.99 102.01) (end 121 100.02) (width 0.2) (layer "F.Cu") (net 12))
 (segment (start 121.03 91.5) (end 121 91.5) (width 0.2) (layer "F.Cu") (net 12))
 (segment (start 158 86) (end 158 88.775) (width 0.2) (layer "F.Cu") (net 12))
 (segment (start 158 88.775) (end 156.275 90.5) (width 0.2) (layer "F.Cu") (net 12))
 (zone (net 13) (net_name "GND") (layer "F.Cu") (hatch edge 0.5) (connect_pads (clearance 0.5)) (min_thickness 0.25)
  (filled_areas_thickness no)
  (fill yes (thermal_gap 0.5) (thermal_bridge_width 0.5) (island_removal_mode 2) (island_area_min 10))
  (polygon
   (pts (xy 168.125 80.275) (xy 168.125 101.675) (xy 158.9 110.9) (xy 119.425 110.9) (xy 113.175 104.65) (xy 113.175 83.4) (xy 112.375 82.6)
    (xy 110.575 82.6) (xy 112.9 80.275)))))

